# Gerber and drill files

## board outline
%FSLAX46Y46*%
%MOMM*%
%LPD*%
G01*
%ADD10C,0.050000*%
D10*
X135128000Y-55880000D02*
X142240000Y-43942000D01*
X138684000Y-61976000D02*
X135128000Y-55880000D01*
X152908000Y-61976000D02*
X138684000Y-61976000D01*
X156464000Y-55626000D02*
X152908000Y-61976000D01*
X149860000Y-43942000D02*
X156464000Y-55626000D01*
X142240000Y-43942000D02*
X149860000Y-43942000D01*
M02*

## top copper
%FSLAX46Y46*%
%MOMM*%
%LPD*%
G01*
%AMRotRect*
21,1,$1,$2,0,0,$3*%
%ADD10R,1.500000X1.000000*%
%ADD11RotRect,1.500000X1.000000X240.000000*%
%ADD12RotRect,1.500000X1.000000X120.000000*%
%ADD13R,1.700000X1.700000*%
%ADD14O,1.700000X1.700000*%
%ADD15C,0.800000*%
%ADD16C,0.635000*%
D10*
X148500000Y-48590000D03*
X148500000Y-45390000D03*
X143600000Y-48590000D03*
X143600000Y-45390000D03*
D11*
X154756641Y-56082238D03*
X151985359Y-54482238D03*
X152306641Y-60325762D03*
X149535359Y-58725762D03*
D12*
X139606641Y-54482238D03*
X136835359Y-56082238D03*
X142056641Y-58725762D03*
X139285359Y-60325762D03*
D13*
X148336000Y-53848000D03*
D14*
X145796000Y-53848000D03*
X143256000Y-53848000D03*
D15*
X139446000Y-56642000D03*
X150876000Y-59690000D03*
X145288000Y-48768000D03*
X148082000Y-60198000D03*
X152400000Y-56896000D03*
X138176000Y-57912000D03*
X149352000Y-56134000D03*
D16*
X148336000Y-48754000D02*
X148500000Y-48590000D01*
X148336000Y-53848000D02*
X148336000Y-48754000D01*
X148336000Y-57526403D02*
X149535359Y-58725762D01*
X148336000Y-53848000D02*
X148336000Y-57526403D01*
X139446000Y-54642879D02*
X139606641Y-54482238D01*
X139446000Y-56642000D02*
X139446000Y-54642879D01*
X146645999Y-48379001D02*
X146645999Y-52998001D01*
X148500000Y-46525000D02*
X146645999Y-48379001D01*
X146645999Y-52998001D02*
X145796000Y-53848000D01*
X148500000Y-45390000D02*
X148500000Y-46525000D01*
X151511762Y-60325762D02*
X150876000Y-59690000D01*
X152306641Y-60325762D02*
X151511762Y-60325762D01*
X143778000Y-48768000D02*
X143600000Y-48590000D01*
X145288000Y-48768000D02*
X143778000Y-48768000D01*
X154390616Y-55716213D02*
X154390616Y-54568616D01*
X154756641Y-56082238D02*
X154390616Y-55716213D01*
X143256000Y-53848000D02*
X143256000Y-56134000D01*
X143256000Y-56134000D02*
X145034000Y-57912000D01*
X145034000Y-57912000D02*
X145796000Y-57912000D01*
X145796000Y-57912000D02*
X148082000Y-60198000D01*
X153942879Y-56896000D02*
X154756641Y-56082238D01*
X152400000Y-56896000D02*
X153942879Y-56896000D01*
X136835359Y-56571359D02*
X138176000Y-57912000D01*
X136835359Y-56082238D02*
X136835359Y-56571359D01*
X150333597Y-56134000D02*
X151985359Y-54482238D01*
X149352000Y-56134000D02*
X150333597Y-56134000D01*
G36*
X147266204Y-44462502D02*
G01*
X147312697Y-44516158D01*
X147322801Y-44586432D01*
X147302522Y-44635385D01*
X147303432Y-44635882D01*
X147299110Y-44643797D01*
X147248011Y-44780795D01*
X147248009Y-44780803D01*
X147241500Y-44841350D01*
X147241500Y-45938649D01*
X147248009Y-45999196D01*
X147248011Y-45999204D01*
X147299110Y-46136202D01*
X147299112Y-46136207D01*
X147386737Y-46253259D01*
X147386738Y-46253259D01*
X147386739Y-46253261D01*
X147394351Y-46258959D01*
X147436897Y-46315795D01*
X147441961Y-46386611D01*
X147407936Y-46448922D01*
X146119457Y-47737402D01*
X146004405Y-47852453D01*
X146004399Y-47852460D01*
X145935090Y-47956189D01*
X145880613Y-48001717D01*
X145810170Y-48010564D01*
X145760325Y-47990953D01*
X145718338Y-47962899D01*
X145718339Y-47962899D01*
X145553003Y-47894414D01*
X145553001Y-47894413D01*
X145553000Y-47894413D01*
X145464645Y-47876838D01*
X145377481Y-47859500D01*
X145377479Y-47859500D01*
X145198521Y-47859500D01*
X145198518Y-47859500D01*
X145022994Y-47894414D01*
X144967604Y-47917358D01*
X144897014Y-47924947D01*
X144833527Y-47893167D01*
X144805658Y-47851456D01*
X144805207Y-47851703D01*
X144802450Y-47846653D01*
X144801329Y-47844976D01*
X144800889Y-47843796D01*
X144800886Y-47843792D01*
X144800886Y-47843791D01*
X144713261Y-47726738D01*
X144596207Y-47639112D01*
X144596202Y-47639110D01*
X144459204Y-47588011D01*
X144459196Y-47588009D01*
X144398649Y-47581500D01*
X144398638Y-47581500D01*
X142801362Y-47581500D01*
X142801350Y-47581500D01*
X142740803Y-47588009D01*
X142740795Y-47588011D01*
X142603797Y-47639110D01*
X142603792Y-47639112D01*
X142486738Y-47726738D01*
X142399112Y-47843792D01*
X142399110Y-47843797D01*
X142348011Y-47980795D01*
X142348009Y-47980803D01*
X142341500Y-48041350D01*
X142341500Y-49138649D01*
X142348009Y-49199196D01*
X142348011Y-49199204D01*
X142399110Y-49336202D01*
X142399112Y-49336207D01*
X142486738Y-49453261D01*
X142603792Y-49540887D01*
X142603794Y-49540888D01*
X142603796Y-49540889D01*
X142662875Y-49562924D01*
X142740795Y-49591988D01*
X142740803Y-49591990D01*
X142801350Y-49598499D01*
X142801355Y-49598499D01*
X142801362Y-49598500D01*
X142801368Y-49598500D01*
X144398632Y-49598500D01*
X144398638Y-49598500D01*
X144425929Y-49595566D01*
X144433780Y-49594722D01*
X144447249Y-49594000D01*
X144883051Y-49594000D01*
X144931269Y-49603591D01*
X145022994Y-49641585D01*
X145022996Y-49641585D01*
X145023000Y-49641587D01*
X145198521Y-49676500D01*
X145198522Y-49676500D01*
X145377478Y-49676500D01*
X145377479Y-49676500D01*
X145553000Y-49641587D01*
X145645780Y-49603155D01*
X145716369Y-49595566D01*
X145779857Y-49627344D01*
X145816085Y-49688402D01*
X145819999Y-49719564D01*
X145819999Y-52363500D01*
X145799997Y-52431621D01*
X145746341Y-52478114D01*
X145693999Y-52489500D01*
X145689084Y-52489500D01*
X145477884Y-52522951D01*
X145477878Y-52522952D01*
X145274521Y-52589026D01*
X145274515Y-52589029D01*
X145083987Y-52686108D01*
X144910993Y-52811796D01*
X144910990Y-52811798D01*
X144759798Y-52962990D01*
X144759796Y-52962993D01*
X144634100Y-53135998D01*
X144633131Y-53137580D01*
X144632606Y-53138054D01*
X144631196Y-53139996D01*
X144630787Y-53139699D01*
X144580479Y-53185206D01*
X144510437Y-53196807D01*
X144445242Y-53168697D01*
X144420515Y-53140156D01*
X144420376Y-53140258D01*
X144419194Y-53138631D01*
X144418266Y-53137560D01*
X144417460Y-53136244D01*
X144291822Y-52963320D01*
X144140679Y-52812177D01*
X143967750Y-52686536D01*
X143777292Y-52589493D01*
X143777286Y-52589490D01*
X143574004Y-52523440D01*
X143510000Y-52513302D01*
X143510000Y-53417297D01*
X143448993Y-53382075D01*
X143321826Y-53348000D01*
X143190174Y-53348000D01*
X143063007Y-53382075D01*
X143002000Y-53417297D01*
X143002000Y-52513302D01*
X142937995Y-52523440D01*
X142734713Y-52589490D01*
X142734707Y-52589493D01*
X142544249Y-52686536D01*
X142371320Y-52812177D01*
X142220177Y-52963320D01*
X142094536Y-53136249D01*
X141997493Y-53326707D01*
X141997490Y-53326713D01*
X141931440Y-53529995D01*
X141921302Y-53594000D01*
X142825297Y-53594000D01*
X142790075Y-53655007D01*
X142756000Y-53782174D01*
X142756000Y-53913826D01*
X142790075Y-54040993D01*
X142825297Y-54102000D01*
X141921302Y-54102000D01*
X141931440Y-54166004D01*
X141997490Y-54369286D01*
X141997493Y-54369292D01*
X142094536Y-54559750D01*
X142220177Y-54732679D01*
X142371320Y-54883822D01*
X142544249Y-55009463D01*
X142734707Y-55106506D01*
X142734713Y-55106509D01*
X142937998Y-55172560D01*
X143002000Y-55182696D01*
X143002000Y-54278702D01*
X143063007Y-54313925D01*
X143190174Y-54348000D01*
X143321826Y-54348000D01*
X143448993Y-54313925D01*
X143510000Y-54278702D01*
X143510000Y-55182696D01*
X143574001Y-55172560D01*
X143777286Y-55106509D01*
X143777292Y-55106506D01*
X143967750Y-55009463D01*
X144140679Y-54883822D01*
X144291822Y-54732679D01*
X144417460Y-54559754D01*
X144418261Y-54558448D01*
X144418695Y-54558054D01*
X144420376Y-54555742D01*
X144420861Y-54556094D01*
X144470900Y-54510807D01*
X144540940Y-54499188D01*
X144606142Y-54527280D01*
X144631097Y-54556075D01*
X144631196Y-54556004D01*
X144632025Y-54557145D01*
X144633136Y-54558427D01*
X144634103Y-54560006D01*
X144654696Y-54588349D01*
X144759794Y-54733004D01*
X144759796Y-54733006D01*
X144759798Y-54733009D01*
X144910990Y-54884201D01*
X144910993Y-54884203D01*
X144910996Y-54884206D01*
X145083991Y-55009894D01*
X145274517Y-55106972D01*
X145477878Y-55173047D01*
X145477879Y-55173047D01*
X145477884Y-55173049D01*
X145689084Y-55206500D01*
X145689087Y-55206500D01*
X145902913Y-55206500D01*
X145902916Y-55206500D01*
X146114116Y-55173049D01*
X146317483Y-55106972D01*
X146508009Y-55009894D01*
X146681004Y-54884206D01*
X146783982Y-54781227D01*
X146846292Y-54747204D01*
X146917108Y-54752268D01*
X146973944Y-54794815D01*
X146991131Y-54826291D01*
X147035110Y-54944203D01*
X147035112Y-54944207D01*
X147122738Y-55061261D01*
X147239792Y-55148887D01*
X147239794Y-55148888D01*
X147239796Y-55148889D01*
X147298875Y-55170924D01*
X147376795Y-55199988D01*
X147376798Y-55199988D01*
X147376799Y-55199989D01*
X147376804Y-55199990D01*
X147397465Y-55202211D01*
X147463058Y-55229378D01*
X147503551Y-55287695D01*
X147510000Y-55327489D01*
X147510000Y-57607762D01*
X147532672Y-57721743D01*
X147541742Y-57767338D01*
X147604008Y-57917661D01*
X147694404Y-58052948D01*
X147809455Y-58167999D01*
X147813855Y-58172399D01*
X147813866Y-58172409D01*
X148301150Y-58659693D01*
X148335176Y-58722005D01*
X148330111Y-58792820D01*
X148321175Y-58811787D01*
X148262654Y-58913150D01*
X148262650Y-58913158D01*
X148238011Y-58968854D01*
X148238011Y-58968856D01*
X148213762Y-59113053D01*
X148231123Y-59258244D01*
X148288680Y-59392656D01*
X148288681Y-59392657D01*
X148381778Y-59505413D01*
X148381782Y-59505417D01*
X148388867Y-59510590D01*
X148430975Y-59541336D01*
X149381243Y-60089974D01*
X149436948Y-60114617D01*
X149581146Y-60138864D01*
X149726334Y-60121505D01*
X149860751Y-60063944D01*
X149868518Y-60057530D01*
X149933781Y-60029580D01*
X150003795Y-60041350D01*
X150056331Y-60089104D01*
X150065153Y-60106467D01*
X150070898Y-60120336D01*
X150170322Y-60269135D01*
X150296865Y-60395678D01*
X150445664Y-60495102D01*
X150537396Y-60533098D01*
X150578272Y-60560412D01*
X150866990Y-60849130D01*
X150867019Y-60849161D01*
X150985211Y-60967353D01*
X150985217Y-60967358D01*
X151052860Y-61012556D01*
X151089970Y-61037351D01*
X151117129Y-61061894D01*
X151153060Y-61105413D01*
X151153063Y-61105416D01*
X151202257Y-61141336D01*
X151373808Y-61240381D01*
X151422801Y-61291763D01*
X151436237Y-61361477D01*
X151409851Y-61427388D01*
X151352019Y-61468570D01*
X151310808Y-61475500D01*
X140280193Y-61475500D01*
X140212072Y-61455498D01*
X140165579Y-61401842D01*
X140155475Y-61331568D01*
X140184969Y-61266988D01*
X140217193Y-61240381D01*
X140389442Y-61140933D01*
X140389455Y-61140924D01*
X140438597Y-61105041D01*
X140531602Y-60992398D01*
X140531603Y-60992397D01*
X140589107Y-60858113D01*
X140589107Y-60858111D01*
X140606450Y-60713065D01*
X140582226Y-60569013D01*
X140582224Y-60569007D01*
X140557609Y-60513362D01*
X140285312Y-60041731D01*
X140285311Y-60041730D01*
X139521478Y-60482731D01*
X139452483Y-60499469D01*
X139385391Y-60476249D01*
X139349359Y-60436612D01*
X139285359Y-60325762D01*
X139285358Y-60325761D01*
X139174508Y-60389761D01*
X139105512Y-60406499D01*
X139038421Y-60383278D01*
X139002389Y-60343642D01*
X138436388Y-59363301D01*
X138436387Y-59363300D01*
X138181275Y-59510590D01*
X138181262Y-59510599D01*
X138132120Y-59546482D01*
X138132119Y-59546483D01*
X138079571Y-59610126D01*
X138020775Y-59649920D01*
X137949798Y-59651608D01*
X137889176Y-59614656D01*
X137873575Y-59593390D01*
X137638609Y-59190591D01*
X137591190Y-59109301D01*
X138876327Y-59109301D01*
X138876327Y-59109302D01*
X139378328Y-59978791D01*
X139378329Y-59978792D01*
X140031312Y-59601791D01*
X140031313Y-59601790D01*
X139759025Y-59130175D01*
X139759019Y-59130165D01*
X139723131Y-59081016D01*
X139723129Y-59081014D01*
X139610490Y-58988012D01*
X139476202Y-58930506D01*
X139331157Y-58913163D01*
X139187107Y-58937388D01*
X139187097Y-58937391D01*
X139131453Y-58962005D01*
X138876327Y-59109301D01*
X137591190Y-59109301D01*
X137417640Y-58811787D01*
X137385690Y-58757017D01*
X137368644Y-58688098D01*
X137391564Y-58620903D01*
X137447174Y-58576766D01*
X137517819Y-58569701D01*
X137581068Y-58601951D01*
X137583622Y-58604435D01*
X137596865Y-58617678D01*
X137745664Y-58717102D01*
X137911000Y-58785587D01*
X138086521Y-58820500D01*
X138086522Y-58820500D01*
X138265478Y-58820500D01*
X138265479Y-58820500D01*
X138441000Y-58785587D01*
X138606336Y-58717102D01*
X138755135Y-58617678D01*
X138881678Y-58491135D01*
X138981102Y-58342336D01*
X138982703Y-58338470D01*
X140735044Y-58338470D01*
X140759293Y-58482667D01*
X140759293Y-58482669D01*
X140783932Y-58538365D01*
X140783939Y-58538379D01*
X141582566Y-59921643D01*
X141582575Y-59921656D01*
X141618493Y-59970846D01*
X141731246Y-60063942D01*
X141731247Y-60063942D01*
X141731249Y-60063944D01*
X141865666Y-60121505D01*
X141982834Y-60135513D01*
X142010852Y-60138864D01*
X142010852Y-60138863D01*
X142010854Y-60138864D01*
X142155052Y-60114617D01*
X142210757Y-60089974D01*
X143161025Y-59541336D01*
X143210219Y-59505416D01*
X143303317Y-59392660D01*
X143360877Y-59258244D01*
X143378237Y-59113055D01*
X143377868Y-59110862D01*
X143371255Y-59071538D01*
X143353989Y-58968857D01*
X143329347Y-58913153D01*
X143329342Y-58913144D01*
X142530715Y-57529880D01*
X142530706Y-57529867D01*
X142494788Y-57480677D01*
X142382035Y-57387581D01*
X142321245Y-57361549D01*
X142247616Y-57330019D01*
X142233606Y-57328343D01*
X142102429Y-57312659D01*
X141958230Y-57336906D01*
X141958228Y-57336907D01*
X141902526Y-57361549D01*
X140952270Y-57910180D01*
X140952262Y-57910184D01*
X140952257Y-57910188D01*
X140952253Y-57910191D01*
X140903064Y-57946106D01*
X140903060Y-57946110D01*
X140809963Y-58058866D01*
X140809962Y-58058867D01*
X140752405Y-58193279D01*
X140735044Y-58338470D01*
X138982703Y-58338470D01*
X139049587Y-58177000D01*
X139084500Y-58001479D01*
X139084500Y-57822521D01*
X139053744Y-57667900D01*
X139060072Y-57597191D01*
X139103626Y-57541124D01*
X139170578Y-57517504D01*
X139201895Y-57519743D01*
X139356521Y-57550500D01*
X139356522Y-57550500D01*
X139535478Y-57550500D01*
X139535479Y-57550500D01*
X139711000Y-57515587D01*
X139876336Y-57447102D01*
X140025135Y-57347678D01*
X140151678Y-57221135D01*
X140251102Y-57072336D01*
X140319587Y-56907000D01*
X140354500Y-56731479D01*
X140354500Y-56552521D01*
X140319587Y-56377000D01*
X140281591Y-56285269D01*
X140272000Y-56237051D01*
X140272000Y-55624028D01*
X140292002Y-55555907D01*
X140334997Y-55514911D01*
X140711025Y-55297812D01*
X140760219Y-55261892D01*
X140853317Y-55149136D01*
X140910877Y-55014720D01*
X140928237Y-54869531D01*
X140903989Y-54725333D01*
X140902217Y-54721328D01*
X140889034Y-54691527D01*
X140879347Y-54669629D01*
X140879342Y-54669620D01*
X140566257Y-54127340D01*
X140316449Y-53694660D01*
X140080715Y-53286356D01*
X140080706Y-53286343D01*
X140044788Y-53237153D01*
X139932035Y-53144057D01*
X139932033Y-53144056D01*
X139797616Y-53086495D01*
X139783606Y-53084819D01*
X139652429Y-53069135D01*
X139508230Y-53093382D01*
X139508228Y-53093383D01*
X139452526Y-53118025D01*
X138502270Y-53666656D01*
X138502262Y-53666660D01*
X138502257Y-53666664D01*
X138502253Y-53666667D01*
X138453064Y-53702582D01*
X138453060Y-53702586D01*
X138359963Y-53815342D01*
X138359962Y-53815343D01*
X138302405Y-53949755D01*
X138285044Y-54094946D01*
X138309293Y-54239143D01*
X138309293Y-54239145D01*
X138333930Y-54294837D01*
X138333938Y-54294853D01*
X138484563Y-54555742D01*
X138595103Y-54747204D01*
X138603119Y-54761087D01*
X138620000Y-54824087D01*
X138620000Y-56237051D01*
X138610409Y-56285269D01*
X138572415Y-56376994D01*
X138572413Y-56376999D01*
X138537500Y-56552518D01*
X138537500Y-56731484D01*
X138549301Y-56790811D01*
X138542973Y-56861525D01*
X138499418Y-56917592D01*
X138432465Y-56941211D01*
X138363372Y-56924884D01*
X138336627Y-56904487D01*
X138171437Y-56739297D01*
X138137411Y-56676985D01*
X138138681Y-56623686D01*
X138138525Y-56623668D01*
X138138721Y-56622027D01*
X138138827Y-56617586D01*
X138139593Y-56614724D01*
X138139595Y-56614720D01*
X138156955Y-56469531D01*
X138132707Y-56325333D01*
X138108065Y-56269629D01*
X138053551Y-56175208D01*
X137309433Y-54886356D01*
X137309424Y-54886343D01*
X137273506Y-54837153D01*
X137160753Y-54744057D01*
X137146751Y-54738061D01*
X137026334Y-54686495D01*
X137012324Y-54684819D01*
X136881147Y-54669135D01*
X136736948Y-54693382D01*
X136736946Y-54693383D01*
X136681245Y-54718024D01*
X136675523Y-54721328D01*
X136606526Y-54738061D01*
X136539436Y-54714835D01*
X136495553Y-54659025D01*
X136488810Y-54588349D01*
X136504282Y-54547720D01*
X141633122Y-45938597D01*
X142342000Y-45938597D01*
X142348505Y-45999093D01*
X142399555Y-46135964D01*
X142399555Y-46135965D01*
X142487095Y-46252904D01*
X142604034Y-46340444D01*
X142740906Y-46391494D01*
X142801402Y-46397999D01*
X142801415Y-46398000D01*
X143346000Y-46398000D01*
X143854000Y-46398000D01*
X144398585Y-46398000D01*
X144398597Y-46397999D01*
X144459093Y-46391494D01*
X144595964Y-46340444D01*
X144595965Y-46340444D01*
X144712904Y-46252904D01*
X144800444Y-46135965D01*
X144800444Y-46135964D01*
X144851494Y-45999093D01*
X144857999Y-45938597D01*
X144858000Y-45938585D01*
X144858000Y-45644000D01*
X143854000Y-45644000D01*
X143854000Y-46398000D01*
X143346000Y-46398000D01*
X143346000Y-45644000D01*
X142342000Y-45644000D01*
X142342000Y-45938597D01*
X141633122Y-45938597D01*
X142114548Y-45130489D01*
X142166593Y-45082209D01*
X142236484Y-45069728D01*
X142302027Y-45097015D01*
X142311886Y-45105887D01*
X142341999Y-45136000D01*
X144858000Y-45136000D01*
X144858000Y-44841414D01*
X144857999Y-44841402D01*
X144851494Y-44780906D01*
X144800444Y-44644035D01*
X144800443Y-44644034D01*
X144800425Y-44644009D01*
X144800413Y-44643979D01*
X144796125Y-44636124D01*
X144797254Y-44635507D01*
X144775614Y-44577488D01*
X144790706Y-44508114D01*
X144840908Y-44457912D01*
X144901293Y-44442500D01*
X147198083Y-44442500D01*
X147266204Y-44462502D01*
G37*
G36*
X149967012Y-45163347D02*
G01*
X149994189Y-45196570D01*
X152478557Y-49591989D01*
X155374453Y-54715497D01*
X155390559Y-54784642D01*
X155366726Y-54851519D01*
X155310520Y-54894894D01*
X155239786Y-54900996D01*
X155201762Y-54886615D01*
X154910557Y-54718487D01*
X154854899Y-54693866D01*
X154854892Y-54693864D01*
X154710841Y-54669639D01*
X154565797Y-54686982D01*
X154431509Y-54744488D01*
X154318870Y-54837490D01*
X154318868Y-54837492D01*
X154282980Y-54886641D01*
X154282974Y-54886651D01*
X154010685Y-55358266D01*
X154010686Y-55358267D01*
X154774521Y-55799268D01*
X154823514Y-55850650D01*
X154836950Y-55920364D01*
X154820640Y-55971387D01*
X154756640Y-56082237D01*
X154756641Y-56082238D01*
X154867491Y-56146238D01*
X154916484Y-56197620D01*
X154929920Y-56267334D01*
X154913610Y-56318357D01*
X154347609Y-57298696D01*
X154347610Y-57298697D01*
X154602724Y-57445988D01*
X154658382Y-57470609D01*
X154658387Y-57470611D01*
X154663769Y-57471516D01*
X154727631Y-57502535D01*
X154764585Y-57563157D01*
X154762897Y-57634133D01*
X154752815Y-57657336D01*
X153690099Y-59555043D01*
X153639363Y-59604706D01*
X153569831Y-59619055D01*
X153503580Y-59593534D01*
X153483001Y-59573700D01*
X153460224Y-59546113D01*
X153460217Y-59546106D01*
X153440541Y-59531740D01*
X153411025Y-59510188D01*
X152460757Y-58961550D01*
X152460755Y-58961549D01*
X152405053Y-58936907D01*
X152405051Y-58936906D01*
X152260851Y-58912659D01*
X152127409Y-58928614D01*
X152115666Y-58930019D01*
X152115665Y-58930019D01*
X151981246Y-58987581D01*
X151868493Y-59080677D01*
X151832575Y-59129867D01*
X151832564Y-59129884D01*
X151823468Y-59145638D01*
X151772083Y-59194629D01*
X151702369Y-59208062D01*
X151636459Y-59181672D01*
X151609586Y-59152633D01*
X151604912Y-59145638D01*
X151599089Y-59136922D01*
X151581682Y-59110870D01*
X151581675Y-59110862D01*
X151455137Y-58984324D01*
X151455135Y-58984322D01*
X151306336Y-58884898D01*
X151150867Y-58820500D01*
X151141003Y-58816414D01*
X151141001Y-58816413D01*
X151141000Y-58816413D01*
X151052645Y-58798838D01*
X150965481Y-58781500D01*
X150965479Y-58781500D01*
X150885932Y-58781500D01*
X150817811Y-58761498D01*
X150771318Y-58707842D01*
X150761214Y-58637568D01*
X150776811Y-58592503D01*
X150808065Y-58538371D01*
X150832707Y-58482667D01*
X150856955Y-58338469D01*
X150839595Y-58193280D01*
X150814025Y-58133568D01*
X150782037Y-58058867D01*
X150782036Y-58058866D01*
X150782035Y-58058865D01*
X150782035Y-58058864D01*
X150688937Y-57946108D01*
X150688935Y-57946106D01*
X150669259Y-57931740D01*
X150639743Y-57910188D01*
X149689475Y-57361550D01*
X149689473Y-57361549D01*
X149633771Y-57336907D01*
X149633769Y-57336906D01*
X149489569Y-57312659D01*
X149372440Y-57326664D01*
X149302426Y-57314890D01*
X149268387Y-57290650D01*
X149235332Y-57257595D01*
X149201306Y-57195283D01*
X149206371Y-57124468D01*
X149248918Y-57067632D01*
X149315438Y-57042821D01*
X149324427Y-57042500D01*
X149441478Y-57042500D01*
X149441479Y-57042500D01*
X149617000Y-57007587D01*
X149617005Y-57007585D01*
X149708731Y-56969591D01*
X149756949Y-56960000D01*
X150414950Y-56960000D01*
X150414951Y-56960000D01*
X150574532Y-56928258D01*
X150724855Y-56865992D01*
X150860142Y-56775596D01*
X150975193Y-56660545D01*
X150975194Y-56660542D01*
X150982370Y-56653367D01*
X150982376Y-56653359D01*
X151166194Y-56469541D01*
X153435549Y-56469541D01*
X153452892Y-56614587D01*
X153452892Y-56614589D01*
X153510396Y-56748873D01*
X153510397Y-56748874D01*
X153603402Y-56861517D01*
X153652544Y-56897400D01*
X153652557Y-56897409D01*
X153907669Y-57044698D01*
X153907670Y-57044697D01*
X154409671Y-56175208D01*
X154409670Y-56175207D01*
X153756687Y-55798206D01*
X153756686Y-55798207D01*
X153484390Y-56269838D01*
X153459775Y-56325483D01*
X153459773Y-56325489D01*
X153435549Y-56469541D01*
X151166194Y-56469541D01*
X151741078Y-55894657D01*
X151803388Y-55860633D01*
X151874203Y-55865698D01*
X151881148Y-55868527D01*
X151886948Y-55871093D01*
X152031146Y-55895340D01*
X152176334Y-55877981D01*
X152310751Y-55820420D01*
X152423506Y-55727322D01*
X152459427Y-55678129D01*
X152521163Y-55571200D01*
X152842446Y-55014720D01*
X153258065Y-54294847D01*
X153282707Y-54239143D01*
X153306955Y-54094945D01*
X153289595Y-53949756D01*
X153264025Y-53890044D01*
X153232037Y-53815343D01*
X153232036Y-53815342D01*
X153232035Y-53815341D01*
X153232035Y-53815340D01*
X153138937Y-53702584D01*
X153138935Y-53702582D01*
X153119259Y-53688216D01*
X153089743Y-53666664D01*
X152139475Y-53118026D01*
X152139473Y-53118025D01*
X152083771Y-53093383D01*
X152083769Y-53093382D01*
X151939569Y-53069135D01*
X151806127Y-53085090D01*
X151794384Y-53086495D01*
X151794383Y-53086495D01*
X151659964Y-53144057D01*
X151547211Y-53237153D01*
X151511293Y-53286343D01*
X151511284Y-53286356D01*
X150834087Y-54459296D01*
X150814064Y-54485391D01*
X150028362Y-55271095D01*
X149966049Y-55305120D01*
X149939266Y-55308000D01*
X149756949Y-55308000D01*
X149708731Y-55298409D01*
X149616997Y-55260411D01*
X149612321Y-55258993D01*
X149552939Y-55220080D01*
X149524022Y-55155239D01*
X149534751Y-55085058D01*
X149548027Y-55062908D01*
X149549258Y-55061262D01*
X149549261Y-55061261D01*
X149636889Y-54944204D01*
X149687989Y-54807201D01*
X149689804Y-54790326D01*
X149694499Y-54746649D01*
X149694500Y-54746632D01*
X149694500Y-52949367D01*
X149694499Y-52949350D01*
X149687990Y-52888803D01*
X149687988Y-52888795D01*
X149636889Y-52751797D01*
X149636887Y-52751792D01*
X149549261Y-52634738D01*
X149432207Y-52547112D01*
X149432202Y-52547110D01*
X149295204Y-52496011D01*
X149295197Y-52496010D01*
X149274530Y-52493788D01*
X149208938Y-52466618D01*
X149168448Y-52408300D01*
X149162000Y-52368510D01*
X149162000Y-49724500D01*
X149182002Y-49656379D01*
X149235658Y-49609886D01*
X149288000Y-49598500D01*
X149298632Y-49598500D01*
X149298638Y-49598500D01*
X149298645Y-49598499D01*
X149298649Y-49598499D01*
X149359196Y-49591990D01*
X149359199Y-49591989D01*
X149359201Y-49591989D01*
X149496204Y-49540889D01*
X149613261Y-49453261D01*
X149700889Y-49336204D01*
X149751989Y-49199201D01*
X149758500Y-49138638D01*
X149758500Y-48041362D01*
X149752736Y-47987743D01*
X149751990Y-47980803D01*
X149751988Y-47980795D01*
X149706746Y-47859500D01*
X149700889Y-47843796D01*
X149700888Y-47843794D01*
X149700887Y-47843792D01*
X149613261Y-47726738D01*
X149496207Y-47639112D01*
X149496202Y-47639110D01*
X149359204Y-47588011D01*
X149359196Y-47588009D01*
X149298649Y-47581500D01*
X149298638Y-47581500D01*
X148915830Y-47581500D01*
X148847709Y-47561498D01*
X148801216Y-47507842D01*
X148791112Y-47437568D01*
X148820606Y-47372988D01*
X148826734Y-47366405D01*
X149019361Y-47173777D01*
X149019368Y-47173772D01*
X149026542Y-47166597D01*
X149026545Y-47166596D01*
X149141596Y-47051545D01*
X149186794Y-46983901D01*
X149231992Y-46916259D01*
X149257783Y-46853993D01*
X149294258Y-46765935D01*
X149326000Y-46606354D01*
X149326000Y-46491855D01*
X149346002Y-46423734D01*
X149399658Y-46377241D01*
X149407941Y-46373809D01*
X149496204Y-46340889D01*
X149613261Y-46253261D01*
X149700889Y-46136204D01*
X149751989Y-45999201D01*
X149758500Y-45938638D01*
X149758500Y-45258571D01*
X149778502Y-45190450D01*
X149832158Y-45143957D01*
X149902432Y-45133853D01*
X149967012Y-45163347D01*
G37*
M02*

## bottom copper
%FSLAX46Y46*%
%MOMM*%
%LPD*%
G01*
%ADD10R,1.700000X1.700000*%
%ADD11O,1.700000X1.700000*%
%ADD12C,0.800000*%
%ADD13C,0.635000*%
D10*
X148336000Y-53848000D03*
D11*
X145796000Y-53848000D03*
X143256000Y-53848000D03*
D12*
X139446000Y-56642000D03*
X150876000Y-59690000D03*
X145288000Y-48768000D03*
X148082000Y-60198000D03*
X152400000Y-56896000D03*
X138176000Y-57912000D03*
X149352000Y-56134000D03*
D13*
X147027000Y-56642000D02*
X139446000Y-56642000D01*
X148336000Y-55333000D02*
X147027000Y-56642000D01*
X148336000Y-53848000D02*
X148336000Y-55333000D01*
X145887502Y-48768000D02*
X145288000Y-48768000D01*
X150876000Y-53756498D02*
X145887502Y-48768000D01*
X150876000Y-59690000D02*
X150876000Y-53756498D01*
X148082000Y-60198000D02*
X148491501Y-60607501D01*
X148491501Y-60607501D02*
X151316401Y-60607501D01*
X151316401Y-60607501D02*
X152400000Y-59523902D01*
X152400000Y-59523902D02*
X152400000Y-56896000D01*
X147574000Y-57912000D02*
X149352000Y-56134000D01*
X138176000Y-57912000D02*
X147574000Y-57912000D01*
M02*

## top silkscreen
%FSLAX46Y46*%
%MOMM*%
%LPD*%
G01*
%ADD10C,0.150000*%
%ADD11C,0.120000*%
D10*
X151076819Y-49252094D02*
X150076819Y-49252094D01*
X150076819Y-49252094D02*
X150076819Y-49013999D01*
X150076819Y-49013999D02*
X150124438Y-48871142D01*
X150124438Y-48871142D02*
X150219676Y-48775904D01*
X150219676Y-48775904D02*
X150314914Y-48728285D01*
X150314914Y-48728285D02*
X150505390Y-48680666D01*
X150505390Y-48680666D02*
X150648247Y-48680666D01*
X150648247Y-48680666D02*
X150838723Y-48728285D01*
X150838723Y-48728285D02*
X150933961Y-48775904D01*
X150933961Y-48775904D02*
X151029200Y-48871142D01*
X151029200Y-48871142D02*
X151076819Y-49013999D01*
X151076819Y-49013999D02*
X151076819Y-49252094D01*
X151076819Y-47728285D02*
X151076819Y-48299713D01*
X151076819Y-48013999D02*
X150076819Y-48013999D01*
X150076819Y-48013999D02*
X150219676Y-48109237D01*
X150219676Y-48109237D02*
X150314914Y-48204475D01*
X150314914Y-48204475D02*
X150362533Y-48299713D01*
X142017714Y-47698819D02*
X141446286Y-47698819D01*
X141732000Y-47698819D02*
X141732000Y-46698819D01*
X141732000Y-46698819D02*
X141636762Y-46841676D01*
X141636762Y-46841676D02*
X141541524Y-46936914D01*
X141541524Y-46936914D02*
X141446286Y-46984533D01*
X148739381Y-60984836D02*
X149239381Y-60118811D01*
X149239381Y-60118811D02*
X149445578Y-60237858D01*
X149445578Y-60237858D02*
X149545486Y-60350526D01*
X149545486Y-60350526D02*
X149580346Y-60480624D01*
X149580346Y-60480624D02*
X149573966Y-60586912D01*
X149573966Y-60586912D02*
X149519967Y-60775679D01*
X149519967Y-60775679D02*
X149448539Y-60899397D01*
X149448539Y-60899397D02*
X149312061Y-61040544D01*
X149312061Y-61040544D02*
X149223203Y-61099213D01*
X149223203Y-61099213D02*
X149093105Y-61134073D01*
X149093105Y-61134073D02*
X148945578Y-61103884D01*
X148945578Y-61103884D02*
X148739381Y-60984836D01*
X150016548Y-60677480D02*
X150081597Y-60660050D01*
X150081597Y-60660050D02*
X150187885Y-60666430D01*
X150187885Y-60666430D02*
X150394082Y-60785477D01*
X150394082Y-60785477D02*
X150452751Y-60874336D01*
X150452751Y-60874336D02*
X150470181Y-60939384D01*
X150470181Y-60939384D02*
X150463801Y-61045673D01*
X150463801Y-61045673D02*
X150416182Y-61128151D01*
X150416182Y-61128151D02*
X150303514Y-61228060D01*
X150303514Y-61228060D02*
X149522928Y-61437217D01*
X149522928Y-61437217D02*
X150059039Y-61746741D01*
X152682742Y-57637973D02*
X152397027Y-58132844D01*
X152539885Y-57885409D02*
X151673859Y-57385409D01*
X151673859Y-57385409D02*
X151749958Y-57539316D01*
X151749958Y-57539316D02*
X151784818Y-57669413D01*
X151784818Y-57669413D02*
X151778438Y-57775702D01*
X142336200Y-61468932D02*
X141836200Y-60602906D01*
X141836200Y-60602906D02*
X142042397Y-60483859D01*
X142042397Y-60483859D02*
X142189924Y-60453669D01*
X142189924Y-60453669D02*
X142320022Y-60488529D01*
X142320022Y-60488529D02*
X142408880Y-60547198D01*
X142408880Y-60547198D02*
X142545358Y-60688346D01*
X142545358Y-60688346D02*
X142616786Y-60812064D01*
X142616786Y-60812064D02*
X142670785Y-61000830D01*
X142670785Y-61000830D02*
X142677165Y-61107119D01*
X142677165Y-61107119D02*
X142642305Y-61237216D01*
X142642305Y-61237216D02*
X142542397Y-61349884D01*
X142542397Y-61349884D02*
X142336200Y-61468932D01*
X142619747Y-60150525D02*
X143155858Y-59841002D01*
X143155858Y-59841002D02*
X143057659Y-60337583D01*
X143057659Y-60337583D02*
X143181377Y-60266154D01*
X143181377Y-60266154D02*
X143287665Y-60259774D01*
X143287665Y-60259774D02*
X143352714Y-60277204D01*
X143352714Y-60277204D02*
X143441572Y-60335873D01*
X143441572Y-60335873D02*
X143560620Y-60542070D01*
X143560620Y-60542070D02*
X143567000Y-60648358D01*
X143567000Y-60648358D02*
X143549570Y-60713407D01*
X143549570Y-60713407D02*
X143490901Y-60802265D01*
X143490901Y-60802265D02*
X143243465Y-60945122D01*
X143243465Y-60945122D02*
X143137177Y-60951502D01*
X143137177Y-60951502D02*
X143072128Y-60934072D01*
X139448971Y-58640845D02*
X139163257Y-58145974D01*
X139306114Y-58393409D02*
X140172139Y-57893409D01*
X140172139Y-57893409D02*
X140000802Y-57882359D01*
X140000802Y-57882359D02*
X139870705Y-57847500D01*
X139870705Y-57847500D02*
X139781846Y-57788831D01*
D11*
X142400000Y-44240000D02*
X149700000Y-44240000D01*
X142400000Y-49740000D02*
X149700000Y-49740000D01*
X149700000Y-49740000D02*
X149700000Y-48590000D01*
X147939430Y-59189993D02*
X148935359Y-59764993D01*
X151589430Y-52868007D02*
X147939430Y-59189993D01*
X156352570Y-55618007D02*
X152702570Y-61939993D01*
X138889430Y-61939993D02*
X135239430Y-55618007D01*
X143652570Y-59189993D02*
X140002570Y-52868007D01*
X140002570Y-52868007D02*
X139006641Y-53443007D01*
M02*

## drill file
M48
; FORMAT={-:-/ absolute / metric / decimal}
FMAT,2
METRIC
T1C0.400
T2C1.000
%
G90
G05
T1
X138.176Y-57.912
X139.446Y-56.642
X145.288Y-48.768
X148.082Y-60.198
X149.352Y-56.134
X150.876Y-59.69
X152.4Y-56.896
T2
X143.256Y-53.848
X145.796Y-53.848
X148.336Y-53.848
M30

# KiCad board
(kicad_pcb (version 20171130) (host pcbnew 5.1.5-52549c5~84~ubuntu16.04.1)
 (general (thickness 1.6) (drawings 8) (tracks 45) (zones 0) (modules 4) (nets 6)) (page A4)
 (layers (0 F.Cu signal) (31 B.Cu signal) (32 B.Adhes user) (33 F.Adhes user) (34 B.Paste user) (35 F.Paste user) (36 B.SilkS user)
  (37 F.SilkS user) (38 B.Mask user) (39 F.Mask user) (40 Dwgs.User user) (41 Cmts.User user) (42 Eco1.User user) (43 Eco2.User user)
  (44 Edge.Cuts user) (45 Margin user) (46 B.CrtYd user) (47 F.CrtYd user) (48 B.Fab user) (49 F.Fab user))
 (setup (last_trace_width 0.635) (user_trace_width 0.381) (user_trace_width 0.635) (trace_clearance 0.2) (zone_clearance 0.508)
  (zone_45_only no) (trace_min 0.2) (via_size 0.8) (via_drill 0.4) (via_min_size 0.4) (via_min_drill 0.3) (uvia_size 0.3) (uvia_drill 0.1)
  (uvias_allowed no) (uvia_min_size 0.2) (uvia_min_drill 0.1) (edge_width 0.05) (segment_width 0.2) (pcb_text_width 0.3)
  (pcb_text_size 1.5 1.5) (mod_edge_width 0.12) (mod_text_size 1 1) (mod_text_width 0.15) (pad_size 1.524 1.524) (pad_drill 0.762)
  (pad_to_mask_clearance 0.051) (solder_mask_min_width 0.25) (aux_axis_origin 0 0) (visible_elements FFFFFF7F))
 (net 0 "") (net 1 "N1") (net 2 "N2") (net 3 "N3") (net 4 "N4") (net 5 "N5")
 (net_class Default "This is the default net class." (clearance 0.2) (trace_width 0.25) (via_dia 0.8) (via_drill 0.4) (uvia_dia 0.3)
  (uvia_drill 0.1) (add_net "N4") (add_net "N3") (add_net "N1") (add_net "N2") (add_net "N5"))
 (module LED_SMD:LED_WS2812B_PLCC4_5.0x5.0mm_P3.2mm (layer F.Cu) (at 146.05 46.99)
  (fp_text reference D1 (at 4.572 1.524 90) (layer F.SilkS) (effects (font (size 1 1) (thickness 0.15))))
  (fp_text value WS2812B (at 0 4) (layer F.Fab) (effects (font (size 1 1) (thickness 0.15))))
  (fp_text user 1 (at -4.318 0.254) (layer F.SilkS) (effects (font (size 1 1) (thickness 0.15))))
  (fp_line (start -3.65 -2.75) (end 3.65 -2.75) (layer F.SilkS) (width 0.12))
  (fp_line (start -3.65 2.75) (end 3.65 2.75) (layer F.SilkS) (width 0.12))
  (fp_line (start 3.65 2.75) (end 3.65 1.6) (layer F.SilkS) (width 0.12))
  (pad 3 smd rect (at 2.45 1.6) (size 1.5 1) (layers F.Cu F.Paste F.Mask) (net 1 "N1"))
  (pad 4 smd rect (at 2.45 -1.6) (size 1.5 1) (layers F.Cu F.Paste F.Mask) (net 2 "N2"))
  (pad 2 smd rect (at -2.45 1.6) (size 1.5 1) (layers F.Cu F.Paste F.Mask) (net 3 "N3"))
  (pad 1 smd rect (at -2.45 -1.6) (size 1.5 1) (layers F.Cu F.Paste F.Mask) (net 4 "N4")))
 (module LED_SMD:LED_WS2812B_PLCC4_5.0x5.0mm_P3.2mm (layer F.Cu) (at 152.146 57.404 240)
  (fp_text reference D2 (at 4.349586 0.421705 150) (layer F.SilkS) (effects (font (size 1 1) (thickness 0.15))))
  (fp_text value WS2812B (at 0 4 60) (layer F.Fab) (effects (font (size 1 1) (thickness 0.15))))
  (fp_line (start 3.65 2.75) (end 3.65 1.6) (layer F.SilkS) (width 0.12))
  (fp_line (start -3.65 2.75) (end 3.65 2.75) (layer F.SilkS) (width 0.12))
  (fp_line (start -3.65 -2.75) (end 3.65 -2.75) (layer F.SilkS) (width 0.12))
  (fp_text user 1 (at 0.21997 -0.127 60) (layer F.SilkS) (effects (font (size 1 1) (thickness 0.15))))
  (pad 1 smd rect (at -2.45 -1.6 240) (size 1.5 1) (layers F.Cu F.Paste F.Mask) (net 4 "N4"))
  (pad 2 smd rect (at -2.45 1.6 240) (size 1.5 1) (layers F.Cu F.Paste F.Mask) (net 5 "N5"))
  (pad 4 smd rect (at 2.45 -1.6 240) (size 1.5 1) (layers F.Cu F.Paste F.Mask) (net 3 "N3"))
  (pad 3 smd rect (at 2.45 1.6 240) (size 1.5 1) (layers F.Cu F.Paste F.Mask) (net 1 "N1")))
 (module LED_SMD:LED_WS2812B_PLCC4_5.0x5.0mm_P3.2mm (layer F.Cu) (at 139.446 57.404 120)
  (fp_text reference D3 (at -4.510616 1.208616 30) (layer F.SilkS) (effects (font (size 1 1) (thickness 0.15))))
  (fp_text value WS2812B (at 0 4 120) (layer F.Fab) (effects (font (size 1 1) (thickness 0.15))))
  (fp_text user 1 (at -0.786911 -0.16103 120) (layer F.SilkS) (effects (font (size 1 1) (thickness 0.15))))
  (fp_line (start -3.65 -2.75) (end 3.65 -2.75) (layer F.SilkS) (width 0.12))
  (fp_line (start -3.65 2.75) (end 3.65 2.75) (layer F.SilkS) (width 0.12))
  (fp_line (start 3.65 2.75) (end 3.65 1.6) (layer F.SilkS) (width 0.12))
  (pad 3 smd rect (at 2.45 1.6 120) (size 1.5 1) (layers F.Cu F.Paste F.Mask) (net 1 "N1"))
  (pad 4 smd rect (at 2.45 -1.6 120) (size 1.5 1) (layers F.Cu F.Paste F.Mask) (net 5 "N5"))
  (pad 2 smd rect (at -2.45 1.6 120) (size 1.5 1) (layers F.Cu F.Paste F.Mask))
  (pad 1 smd rect (at -2.45 -1.6 120) (size 1.5 1) (layers F.Cu F.Paste F.Mask) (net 4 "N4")))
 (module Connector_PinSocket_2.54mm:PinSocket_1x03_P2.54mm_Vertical (layer B.Cu) (at 148.336 53.848 90)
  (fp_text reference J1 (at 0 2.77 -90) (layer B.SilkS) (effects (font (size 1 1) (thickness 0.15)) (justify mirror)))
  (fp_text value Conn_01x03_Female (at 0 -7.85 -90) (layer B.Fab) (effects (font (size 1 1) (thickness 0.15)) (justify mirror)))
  (pad 1 thru_hole rect (at 0 0 90) (size 1.7 1.7) (drill 1) (layers *.Cu *.Mask) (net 1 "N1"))
  (pad 2 thru_hole oval (at 0 -2.54 90) (size 1.7 1.7) (drill 1) (layers *.Cu *.Mask) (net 2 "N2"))
  (pad 3 thru_hole oval (at 0 -5.08 90) (size 1.7 1.7) (drill 1) (layers *.Cu *.Mask) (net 4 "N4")))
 (gr_line (start 135.128 55.88) (end 142.24 43.942) (layer Edge.Cuts) (width 0.05))
 (gr_line (start 138.684 61.976) (end 135.128 55.88) (layer Edge.Cuts) (width 0.05))
 (gr_line (start 152.908 61.976) (end 138.684 61.976) (layer Edge.Cuts) (width 0.05))
 (gr_line (start 156.464 55.626) (end 152.908 61.976) (layer Edge.Cuts) (width 0.05))
 (gr_line (start 149.86 43.942) (end 156.464 55.626) (layer Edge.Cuts) (width 0.05))
 (gr_line (start 142.24 43.942) (end 149.86 43.942) (layer Edge.Cuts) (width 0.05))
 (segment (start 148.336 48.754) (end 148.5 48.59) (width 0.635) (layer F.Cu) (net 1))
 (segment (start 148.336 53.848) (end 148.336 48.754) (width 0.635) (layer F.Cu) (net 1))
 (segment (start 148.336 57.526403) (end 149.535359 58.725762) (width 0.635) (layer F.Cu) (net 1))
 (segment (start 148.336 53.848) (end 148.336 57.526403) (width 0.635) (layer F.Cu) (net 1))
 (segment (start 147.027 56.642) (end 139.446 56.642) (width 0.635) (layer B.Cu) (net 1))
 (segment (start 148.336 55.333) (end 147.027 56.642) (width 0.635) (layer B.Cu) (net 1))
 (via (at 139.446 56.642) (size 0.8) (drill 0.4) (layers F.Cu B.Cu) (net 1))
 (segment (start 148.336 53.848) (end 148.336 55.333) (width 0.635) (layer B.Cu) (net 1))
 (segment (start 139.446 54.642879) (end 139.606641 54.482238) (width 0.635) (layer F.Cu) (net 1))
 (segment (start 139.446 56.642) (end 139.446 54.642879) (width 0.635) (layer F.Cu) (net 1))
 (segment (start 146.645999 48.379001) (end 146.645999 52.998001) (width 0.635) (layer F.Cu) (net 2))
 (segment (start 148.5 46.525) (end 146.645999 48.379001) (width 0.635) (layer F.Cu) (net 2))
 (segment (start 146.645999 52.998001) (end 145.796 53.848) (width 0.635) (layer F.Cu) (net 2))
 (segment (start 148.5 45.39) (end 148.5 46.525) (width 0.635) (layer F.Cu) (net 2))
 (segment (start 151.511762 60.325762) (end 150.876 59.69) (width 0.635) (layer F.Cu) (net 3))
 (via (at 150.876 59.69) (size 0.8) (drill 0.4) (layers F.Cu B.Cu) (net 3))
 (segment (start 152.306641 60.325762) (end 151.511762 60.325762) (width 0.635) (layer F.Cu) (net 3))
 (via (at 145.288 48.768) (size 0.8) (drill 0.4) (layers F.Cu B.Cu) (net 3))
 (segment (start 145.887502 48.768) (end 145.288 48.768) (width 0.635) (layer B.Cu) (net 3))
 (segment (start 150.876 53.756498) (end 145.887502 48.768) (width 0.635) (layer B.Cu) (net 3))
 (segment (start 150.876 59.69) (end 150.876 53.756498) (width 0.635) (layer B.Cu) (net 3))
 (segment (start 143.778 48.768) (end 143.6 48.59) (width 0.635) (layer F.Cu) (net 3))
 (segment (start 145.288 48.768) (end 143.778 48.768) (width 0.635) (layer F.Cu) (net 3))
 (segment (start 154.390616 55.716213) (end 154.390616 54.568616) (width 0.635) (layer F.Cu) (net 4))
 (segment (start 154.756641 56.082238) (end 154.390616 55.716213) (width 0.635) (layer F.Cu) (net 4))
 (segment (start 143.256 53.848) (end 143.256 56.134) (width 0.635) (layer F.Cu) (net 4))
 (segment (start 143.256 56.134) (end 145.034 57.912) (width 0.635) (layer F.Cu) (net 4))
 (segment (start 145.034 57.912) (end 145.796 57.912) (width 0.635) (layer F.Cu) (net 4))
 (segment (start 145.796 57.912) (end 148.082 60.198) (width 0.635) (layer F.Cu) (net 4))
 (via (at 148.082 60.198) (size 0.8) (drill 0.4) (layers F.Cu B.Cu) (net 4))
 (segment (start 148.082 60.198) (end 148.491501 60.607501) (width 0.635) (layer B.Cu) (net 4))
 (via (at 152.4 56.896) (size 0.8) (drill 0.4) (layers F.Cu B.Cu) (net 4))
 (segment (start 148.491501 60.607501) (end 151.316401 60.607501) (width 0.635) (layer B.Cu) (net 4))
 (segment (start 151.316401 60.607501) (end 152.4 59.523902) (width 0.635) (layer B.Cu) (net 4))
 (segment (start 152.4 59.523902) (end 152.4 56.896) (width 0.635) (layer B.Cu) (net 4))
 (segment (start 153.942879 56.896) (end 154.756641 56.082238) (width 0.635) (layer F.Cu) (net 4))
 (segment (start 152.4 56.896) (end 153.942879 56.896) (width 0.635) (layer F.Cu) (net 4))
 (via (at 138.176 57.912) (size 0.8) (drill 0.4) (layers F.Cu B.Cu) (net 5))
 (segment (start 136.835359 56.571359) (end 138.176 57.912) (width 0.635) (layer F.Cu) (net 5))
 (segment (start 136.835359 56.082238) (end 136.835359 56.571359) (width 0.635) (layer F.Cu) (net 5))
 (via (at 149.352 56.134) (size 0.8) (drill 0.4) (layers F.Cu B.Cu) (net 5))
 (segment (start 147.574 57.912) (end 149.352 56.134) (width 0.635) (layer B.Cu) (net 5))
 (segment (start 138.176 57.912) (end 147.574 57.912) (width 0.635) (layer B.Cu) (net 5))
 (segment (start 150.333597 56.134) (end 151.985359 54.482238) (width 0.635) (layer F.Cu) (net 5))
 (segment (start 149.352 56.134) (end 150.333597 56.134) (width 0.635) (layer F.Cu) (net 5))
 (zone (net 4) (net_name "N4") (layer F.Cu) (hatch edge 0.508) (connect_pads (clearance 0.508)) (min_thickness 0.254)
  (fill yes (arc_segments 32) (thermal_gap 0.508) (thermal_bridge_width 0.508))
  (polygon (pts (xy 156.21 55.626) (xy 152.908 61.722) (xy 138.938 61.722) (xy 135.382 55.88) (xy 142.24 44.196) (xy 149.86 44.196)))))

